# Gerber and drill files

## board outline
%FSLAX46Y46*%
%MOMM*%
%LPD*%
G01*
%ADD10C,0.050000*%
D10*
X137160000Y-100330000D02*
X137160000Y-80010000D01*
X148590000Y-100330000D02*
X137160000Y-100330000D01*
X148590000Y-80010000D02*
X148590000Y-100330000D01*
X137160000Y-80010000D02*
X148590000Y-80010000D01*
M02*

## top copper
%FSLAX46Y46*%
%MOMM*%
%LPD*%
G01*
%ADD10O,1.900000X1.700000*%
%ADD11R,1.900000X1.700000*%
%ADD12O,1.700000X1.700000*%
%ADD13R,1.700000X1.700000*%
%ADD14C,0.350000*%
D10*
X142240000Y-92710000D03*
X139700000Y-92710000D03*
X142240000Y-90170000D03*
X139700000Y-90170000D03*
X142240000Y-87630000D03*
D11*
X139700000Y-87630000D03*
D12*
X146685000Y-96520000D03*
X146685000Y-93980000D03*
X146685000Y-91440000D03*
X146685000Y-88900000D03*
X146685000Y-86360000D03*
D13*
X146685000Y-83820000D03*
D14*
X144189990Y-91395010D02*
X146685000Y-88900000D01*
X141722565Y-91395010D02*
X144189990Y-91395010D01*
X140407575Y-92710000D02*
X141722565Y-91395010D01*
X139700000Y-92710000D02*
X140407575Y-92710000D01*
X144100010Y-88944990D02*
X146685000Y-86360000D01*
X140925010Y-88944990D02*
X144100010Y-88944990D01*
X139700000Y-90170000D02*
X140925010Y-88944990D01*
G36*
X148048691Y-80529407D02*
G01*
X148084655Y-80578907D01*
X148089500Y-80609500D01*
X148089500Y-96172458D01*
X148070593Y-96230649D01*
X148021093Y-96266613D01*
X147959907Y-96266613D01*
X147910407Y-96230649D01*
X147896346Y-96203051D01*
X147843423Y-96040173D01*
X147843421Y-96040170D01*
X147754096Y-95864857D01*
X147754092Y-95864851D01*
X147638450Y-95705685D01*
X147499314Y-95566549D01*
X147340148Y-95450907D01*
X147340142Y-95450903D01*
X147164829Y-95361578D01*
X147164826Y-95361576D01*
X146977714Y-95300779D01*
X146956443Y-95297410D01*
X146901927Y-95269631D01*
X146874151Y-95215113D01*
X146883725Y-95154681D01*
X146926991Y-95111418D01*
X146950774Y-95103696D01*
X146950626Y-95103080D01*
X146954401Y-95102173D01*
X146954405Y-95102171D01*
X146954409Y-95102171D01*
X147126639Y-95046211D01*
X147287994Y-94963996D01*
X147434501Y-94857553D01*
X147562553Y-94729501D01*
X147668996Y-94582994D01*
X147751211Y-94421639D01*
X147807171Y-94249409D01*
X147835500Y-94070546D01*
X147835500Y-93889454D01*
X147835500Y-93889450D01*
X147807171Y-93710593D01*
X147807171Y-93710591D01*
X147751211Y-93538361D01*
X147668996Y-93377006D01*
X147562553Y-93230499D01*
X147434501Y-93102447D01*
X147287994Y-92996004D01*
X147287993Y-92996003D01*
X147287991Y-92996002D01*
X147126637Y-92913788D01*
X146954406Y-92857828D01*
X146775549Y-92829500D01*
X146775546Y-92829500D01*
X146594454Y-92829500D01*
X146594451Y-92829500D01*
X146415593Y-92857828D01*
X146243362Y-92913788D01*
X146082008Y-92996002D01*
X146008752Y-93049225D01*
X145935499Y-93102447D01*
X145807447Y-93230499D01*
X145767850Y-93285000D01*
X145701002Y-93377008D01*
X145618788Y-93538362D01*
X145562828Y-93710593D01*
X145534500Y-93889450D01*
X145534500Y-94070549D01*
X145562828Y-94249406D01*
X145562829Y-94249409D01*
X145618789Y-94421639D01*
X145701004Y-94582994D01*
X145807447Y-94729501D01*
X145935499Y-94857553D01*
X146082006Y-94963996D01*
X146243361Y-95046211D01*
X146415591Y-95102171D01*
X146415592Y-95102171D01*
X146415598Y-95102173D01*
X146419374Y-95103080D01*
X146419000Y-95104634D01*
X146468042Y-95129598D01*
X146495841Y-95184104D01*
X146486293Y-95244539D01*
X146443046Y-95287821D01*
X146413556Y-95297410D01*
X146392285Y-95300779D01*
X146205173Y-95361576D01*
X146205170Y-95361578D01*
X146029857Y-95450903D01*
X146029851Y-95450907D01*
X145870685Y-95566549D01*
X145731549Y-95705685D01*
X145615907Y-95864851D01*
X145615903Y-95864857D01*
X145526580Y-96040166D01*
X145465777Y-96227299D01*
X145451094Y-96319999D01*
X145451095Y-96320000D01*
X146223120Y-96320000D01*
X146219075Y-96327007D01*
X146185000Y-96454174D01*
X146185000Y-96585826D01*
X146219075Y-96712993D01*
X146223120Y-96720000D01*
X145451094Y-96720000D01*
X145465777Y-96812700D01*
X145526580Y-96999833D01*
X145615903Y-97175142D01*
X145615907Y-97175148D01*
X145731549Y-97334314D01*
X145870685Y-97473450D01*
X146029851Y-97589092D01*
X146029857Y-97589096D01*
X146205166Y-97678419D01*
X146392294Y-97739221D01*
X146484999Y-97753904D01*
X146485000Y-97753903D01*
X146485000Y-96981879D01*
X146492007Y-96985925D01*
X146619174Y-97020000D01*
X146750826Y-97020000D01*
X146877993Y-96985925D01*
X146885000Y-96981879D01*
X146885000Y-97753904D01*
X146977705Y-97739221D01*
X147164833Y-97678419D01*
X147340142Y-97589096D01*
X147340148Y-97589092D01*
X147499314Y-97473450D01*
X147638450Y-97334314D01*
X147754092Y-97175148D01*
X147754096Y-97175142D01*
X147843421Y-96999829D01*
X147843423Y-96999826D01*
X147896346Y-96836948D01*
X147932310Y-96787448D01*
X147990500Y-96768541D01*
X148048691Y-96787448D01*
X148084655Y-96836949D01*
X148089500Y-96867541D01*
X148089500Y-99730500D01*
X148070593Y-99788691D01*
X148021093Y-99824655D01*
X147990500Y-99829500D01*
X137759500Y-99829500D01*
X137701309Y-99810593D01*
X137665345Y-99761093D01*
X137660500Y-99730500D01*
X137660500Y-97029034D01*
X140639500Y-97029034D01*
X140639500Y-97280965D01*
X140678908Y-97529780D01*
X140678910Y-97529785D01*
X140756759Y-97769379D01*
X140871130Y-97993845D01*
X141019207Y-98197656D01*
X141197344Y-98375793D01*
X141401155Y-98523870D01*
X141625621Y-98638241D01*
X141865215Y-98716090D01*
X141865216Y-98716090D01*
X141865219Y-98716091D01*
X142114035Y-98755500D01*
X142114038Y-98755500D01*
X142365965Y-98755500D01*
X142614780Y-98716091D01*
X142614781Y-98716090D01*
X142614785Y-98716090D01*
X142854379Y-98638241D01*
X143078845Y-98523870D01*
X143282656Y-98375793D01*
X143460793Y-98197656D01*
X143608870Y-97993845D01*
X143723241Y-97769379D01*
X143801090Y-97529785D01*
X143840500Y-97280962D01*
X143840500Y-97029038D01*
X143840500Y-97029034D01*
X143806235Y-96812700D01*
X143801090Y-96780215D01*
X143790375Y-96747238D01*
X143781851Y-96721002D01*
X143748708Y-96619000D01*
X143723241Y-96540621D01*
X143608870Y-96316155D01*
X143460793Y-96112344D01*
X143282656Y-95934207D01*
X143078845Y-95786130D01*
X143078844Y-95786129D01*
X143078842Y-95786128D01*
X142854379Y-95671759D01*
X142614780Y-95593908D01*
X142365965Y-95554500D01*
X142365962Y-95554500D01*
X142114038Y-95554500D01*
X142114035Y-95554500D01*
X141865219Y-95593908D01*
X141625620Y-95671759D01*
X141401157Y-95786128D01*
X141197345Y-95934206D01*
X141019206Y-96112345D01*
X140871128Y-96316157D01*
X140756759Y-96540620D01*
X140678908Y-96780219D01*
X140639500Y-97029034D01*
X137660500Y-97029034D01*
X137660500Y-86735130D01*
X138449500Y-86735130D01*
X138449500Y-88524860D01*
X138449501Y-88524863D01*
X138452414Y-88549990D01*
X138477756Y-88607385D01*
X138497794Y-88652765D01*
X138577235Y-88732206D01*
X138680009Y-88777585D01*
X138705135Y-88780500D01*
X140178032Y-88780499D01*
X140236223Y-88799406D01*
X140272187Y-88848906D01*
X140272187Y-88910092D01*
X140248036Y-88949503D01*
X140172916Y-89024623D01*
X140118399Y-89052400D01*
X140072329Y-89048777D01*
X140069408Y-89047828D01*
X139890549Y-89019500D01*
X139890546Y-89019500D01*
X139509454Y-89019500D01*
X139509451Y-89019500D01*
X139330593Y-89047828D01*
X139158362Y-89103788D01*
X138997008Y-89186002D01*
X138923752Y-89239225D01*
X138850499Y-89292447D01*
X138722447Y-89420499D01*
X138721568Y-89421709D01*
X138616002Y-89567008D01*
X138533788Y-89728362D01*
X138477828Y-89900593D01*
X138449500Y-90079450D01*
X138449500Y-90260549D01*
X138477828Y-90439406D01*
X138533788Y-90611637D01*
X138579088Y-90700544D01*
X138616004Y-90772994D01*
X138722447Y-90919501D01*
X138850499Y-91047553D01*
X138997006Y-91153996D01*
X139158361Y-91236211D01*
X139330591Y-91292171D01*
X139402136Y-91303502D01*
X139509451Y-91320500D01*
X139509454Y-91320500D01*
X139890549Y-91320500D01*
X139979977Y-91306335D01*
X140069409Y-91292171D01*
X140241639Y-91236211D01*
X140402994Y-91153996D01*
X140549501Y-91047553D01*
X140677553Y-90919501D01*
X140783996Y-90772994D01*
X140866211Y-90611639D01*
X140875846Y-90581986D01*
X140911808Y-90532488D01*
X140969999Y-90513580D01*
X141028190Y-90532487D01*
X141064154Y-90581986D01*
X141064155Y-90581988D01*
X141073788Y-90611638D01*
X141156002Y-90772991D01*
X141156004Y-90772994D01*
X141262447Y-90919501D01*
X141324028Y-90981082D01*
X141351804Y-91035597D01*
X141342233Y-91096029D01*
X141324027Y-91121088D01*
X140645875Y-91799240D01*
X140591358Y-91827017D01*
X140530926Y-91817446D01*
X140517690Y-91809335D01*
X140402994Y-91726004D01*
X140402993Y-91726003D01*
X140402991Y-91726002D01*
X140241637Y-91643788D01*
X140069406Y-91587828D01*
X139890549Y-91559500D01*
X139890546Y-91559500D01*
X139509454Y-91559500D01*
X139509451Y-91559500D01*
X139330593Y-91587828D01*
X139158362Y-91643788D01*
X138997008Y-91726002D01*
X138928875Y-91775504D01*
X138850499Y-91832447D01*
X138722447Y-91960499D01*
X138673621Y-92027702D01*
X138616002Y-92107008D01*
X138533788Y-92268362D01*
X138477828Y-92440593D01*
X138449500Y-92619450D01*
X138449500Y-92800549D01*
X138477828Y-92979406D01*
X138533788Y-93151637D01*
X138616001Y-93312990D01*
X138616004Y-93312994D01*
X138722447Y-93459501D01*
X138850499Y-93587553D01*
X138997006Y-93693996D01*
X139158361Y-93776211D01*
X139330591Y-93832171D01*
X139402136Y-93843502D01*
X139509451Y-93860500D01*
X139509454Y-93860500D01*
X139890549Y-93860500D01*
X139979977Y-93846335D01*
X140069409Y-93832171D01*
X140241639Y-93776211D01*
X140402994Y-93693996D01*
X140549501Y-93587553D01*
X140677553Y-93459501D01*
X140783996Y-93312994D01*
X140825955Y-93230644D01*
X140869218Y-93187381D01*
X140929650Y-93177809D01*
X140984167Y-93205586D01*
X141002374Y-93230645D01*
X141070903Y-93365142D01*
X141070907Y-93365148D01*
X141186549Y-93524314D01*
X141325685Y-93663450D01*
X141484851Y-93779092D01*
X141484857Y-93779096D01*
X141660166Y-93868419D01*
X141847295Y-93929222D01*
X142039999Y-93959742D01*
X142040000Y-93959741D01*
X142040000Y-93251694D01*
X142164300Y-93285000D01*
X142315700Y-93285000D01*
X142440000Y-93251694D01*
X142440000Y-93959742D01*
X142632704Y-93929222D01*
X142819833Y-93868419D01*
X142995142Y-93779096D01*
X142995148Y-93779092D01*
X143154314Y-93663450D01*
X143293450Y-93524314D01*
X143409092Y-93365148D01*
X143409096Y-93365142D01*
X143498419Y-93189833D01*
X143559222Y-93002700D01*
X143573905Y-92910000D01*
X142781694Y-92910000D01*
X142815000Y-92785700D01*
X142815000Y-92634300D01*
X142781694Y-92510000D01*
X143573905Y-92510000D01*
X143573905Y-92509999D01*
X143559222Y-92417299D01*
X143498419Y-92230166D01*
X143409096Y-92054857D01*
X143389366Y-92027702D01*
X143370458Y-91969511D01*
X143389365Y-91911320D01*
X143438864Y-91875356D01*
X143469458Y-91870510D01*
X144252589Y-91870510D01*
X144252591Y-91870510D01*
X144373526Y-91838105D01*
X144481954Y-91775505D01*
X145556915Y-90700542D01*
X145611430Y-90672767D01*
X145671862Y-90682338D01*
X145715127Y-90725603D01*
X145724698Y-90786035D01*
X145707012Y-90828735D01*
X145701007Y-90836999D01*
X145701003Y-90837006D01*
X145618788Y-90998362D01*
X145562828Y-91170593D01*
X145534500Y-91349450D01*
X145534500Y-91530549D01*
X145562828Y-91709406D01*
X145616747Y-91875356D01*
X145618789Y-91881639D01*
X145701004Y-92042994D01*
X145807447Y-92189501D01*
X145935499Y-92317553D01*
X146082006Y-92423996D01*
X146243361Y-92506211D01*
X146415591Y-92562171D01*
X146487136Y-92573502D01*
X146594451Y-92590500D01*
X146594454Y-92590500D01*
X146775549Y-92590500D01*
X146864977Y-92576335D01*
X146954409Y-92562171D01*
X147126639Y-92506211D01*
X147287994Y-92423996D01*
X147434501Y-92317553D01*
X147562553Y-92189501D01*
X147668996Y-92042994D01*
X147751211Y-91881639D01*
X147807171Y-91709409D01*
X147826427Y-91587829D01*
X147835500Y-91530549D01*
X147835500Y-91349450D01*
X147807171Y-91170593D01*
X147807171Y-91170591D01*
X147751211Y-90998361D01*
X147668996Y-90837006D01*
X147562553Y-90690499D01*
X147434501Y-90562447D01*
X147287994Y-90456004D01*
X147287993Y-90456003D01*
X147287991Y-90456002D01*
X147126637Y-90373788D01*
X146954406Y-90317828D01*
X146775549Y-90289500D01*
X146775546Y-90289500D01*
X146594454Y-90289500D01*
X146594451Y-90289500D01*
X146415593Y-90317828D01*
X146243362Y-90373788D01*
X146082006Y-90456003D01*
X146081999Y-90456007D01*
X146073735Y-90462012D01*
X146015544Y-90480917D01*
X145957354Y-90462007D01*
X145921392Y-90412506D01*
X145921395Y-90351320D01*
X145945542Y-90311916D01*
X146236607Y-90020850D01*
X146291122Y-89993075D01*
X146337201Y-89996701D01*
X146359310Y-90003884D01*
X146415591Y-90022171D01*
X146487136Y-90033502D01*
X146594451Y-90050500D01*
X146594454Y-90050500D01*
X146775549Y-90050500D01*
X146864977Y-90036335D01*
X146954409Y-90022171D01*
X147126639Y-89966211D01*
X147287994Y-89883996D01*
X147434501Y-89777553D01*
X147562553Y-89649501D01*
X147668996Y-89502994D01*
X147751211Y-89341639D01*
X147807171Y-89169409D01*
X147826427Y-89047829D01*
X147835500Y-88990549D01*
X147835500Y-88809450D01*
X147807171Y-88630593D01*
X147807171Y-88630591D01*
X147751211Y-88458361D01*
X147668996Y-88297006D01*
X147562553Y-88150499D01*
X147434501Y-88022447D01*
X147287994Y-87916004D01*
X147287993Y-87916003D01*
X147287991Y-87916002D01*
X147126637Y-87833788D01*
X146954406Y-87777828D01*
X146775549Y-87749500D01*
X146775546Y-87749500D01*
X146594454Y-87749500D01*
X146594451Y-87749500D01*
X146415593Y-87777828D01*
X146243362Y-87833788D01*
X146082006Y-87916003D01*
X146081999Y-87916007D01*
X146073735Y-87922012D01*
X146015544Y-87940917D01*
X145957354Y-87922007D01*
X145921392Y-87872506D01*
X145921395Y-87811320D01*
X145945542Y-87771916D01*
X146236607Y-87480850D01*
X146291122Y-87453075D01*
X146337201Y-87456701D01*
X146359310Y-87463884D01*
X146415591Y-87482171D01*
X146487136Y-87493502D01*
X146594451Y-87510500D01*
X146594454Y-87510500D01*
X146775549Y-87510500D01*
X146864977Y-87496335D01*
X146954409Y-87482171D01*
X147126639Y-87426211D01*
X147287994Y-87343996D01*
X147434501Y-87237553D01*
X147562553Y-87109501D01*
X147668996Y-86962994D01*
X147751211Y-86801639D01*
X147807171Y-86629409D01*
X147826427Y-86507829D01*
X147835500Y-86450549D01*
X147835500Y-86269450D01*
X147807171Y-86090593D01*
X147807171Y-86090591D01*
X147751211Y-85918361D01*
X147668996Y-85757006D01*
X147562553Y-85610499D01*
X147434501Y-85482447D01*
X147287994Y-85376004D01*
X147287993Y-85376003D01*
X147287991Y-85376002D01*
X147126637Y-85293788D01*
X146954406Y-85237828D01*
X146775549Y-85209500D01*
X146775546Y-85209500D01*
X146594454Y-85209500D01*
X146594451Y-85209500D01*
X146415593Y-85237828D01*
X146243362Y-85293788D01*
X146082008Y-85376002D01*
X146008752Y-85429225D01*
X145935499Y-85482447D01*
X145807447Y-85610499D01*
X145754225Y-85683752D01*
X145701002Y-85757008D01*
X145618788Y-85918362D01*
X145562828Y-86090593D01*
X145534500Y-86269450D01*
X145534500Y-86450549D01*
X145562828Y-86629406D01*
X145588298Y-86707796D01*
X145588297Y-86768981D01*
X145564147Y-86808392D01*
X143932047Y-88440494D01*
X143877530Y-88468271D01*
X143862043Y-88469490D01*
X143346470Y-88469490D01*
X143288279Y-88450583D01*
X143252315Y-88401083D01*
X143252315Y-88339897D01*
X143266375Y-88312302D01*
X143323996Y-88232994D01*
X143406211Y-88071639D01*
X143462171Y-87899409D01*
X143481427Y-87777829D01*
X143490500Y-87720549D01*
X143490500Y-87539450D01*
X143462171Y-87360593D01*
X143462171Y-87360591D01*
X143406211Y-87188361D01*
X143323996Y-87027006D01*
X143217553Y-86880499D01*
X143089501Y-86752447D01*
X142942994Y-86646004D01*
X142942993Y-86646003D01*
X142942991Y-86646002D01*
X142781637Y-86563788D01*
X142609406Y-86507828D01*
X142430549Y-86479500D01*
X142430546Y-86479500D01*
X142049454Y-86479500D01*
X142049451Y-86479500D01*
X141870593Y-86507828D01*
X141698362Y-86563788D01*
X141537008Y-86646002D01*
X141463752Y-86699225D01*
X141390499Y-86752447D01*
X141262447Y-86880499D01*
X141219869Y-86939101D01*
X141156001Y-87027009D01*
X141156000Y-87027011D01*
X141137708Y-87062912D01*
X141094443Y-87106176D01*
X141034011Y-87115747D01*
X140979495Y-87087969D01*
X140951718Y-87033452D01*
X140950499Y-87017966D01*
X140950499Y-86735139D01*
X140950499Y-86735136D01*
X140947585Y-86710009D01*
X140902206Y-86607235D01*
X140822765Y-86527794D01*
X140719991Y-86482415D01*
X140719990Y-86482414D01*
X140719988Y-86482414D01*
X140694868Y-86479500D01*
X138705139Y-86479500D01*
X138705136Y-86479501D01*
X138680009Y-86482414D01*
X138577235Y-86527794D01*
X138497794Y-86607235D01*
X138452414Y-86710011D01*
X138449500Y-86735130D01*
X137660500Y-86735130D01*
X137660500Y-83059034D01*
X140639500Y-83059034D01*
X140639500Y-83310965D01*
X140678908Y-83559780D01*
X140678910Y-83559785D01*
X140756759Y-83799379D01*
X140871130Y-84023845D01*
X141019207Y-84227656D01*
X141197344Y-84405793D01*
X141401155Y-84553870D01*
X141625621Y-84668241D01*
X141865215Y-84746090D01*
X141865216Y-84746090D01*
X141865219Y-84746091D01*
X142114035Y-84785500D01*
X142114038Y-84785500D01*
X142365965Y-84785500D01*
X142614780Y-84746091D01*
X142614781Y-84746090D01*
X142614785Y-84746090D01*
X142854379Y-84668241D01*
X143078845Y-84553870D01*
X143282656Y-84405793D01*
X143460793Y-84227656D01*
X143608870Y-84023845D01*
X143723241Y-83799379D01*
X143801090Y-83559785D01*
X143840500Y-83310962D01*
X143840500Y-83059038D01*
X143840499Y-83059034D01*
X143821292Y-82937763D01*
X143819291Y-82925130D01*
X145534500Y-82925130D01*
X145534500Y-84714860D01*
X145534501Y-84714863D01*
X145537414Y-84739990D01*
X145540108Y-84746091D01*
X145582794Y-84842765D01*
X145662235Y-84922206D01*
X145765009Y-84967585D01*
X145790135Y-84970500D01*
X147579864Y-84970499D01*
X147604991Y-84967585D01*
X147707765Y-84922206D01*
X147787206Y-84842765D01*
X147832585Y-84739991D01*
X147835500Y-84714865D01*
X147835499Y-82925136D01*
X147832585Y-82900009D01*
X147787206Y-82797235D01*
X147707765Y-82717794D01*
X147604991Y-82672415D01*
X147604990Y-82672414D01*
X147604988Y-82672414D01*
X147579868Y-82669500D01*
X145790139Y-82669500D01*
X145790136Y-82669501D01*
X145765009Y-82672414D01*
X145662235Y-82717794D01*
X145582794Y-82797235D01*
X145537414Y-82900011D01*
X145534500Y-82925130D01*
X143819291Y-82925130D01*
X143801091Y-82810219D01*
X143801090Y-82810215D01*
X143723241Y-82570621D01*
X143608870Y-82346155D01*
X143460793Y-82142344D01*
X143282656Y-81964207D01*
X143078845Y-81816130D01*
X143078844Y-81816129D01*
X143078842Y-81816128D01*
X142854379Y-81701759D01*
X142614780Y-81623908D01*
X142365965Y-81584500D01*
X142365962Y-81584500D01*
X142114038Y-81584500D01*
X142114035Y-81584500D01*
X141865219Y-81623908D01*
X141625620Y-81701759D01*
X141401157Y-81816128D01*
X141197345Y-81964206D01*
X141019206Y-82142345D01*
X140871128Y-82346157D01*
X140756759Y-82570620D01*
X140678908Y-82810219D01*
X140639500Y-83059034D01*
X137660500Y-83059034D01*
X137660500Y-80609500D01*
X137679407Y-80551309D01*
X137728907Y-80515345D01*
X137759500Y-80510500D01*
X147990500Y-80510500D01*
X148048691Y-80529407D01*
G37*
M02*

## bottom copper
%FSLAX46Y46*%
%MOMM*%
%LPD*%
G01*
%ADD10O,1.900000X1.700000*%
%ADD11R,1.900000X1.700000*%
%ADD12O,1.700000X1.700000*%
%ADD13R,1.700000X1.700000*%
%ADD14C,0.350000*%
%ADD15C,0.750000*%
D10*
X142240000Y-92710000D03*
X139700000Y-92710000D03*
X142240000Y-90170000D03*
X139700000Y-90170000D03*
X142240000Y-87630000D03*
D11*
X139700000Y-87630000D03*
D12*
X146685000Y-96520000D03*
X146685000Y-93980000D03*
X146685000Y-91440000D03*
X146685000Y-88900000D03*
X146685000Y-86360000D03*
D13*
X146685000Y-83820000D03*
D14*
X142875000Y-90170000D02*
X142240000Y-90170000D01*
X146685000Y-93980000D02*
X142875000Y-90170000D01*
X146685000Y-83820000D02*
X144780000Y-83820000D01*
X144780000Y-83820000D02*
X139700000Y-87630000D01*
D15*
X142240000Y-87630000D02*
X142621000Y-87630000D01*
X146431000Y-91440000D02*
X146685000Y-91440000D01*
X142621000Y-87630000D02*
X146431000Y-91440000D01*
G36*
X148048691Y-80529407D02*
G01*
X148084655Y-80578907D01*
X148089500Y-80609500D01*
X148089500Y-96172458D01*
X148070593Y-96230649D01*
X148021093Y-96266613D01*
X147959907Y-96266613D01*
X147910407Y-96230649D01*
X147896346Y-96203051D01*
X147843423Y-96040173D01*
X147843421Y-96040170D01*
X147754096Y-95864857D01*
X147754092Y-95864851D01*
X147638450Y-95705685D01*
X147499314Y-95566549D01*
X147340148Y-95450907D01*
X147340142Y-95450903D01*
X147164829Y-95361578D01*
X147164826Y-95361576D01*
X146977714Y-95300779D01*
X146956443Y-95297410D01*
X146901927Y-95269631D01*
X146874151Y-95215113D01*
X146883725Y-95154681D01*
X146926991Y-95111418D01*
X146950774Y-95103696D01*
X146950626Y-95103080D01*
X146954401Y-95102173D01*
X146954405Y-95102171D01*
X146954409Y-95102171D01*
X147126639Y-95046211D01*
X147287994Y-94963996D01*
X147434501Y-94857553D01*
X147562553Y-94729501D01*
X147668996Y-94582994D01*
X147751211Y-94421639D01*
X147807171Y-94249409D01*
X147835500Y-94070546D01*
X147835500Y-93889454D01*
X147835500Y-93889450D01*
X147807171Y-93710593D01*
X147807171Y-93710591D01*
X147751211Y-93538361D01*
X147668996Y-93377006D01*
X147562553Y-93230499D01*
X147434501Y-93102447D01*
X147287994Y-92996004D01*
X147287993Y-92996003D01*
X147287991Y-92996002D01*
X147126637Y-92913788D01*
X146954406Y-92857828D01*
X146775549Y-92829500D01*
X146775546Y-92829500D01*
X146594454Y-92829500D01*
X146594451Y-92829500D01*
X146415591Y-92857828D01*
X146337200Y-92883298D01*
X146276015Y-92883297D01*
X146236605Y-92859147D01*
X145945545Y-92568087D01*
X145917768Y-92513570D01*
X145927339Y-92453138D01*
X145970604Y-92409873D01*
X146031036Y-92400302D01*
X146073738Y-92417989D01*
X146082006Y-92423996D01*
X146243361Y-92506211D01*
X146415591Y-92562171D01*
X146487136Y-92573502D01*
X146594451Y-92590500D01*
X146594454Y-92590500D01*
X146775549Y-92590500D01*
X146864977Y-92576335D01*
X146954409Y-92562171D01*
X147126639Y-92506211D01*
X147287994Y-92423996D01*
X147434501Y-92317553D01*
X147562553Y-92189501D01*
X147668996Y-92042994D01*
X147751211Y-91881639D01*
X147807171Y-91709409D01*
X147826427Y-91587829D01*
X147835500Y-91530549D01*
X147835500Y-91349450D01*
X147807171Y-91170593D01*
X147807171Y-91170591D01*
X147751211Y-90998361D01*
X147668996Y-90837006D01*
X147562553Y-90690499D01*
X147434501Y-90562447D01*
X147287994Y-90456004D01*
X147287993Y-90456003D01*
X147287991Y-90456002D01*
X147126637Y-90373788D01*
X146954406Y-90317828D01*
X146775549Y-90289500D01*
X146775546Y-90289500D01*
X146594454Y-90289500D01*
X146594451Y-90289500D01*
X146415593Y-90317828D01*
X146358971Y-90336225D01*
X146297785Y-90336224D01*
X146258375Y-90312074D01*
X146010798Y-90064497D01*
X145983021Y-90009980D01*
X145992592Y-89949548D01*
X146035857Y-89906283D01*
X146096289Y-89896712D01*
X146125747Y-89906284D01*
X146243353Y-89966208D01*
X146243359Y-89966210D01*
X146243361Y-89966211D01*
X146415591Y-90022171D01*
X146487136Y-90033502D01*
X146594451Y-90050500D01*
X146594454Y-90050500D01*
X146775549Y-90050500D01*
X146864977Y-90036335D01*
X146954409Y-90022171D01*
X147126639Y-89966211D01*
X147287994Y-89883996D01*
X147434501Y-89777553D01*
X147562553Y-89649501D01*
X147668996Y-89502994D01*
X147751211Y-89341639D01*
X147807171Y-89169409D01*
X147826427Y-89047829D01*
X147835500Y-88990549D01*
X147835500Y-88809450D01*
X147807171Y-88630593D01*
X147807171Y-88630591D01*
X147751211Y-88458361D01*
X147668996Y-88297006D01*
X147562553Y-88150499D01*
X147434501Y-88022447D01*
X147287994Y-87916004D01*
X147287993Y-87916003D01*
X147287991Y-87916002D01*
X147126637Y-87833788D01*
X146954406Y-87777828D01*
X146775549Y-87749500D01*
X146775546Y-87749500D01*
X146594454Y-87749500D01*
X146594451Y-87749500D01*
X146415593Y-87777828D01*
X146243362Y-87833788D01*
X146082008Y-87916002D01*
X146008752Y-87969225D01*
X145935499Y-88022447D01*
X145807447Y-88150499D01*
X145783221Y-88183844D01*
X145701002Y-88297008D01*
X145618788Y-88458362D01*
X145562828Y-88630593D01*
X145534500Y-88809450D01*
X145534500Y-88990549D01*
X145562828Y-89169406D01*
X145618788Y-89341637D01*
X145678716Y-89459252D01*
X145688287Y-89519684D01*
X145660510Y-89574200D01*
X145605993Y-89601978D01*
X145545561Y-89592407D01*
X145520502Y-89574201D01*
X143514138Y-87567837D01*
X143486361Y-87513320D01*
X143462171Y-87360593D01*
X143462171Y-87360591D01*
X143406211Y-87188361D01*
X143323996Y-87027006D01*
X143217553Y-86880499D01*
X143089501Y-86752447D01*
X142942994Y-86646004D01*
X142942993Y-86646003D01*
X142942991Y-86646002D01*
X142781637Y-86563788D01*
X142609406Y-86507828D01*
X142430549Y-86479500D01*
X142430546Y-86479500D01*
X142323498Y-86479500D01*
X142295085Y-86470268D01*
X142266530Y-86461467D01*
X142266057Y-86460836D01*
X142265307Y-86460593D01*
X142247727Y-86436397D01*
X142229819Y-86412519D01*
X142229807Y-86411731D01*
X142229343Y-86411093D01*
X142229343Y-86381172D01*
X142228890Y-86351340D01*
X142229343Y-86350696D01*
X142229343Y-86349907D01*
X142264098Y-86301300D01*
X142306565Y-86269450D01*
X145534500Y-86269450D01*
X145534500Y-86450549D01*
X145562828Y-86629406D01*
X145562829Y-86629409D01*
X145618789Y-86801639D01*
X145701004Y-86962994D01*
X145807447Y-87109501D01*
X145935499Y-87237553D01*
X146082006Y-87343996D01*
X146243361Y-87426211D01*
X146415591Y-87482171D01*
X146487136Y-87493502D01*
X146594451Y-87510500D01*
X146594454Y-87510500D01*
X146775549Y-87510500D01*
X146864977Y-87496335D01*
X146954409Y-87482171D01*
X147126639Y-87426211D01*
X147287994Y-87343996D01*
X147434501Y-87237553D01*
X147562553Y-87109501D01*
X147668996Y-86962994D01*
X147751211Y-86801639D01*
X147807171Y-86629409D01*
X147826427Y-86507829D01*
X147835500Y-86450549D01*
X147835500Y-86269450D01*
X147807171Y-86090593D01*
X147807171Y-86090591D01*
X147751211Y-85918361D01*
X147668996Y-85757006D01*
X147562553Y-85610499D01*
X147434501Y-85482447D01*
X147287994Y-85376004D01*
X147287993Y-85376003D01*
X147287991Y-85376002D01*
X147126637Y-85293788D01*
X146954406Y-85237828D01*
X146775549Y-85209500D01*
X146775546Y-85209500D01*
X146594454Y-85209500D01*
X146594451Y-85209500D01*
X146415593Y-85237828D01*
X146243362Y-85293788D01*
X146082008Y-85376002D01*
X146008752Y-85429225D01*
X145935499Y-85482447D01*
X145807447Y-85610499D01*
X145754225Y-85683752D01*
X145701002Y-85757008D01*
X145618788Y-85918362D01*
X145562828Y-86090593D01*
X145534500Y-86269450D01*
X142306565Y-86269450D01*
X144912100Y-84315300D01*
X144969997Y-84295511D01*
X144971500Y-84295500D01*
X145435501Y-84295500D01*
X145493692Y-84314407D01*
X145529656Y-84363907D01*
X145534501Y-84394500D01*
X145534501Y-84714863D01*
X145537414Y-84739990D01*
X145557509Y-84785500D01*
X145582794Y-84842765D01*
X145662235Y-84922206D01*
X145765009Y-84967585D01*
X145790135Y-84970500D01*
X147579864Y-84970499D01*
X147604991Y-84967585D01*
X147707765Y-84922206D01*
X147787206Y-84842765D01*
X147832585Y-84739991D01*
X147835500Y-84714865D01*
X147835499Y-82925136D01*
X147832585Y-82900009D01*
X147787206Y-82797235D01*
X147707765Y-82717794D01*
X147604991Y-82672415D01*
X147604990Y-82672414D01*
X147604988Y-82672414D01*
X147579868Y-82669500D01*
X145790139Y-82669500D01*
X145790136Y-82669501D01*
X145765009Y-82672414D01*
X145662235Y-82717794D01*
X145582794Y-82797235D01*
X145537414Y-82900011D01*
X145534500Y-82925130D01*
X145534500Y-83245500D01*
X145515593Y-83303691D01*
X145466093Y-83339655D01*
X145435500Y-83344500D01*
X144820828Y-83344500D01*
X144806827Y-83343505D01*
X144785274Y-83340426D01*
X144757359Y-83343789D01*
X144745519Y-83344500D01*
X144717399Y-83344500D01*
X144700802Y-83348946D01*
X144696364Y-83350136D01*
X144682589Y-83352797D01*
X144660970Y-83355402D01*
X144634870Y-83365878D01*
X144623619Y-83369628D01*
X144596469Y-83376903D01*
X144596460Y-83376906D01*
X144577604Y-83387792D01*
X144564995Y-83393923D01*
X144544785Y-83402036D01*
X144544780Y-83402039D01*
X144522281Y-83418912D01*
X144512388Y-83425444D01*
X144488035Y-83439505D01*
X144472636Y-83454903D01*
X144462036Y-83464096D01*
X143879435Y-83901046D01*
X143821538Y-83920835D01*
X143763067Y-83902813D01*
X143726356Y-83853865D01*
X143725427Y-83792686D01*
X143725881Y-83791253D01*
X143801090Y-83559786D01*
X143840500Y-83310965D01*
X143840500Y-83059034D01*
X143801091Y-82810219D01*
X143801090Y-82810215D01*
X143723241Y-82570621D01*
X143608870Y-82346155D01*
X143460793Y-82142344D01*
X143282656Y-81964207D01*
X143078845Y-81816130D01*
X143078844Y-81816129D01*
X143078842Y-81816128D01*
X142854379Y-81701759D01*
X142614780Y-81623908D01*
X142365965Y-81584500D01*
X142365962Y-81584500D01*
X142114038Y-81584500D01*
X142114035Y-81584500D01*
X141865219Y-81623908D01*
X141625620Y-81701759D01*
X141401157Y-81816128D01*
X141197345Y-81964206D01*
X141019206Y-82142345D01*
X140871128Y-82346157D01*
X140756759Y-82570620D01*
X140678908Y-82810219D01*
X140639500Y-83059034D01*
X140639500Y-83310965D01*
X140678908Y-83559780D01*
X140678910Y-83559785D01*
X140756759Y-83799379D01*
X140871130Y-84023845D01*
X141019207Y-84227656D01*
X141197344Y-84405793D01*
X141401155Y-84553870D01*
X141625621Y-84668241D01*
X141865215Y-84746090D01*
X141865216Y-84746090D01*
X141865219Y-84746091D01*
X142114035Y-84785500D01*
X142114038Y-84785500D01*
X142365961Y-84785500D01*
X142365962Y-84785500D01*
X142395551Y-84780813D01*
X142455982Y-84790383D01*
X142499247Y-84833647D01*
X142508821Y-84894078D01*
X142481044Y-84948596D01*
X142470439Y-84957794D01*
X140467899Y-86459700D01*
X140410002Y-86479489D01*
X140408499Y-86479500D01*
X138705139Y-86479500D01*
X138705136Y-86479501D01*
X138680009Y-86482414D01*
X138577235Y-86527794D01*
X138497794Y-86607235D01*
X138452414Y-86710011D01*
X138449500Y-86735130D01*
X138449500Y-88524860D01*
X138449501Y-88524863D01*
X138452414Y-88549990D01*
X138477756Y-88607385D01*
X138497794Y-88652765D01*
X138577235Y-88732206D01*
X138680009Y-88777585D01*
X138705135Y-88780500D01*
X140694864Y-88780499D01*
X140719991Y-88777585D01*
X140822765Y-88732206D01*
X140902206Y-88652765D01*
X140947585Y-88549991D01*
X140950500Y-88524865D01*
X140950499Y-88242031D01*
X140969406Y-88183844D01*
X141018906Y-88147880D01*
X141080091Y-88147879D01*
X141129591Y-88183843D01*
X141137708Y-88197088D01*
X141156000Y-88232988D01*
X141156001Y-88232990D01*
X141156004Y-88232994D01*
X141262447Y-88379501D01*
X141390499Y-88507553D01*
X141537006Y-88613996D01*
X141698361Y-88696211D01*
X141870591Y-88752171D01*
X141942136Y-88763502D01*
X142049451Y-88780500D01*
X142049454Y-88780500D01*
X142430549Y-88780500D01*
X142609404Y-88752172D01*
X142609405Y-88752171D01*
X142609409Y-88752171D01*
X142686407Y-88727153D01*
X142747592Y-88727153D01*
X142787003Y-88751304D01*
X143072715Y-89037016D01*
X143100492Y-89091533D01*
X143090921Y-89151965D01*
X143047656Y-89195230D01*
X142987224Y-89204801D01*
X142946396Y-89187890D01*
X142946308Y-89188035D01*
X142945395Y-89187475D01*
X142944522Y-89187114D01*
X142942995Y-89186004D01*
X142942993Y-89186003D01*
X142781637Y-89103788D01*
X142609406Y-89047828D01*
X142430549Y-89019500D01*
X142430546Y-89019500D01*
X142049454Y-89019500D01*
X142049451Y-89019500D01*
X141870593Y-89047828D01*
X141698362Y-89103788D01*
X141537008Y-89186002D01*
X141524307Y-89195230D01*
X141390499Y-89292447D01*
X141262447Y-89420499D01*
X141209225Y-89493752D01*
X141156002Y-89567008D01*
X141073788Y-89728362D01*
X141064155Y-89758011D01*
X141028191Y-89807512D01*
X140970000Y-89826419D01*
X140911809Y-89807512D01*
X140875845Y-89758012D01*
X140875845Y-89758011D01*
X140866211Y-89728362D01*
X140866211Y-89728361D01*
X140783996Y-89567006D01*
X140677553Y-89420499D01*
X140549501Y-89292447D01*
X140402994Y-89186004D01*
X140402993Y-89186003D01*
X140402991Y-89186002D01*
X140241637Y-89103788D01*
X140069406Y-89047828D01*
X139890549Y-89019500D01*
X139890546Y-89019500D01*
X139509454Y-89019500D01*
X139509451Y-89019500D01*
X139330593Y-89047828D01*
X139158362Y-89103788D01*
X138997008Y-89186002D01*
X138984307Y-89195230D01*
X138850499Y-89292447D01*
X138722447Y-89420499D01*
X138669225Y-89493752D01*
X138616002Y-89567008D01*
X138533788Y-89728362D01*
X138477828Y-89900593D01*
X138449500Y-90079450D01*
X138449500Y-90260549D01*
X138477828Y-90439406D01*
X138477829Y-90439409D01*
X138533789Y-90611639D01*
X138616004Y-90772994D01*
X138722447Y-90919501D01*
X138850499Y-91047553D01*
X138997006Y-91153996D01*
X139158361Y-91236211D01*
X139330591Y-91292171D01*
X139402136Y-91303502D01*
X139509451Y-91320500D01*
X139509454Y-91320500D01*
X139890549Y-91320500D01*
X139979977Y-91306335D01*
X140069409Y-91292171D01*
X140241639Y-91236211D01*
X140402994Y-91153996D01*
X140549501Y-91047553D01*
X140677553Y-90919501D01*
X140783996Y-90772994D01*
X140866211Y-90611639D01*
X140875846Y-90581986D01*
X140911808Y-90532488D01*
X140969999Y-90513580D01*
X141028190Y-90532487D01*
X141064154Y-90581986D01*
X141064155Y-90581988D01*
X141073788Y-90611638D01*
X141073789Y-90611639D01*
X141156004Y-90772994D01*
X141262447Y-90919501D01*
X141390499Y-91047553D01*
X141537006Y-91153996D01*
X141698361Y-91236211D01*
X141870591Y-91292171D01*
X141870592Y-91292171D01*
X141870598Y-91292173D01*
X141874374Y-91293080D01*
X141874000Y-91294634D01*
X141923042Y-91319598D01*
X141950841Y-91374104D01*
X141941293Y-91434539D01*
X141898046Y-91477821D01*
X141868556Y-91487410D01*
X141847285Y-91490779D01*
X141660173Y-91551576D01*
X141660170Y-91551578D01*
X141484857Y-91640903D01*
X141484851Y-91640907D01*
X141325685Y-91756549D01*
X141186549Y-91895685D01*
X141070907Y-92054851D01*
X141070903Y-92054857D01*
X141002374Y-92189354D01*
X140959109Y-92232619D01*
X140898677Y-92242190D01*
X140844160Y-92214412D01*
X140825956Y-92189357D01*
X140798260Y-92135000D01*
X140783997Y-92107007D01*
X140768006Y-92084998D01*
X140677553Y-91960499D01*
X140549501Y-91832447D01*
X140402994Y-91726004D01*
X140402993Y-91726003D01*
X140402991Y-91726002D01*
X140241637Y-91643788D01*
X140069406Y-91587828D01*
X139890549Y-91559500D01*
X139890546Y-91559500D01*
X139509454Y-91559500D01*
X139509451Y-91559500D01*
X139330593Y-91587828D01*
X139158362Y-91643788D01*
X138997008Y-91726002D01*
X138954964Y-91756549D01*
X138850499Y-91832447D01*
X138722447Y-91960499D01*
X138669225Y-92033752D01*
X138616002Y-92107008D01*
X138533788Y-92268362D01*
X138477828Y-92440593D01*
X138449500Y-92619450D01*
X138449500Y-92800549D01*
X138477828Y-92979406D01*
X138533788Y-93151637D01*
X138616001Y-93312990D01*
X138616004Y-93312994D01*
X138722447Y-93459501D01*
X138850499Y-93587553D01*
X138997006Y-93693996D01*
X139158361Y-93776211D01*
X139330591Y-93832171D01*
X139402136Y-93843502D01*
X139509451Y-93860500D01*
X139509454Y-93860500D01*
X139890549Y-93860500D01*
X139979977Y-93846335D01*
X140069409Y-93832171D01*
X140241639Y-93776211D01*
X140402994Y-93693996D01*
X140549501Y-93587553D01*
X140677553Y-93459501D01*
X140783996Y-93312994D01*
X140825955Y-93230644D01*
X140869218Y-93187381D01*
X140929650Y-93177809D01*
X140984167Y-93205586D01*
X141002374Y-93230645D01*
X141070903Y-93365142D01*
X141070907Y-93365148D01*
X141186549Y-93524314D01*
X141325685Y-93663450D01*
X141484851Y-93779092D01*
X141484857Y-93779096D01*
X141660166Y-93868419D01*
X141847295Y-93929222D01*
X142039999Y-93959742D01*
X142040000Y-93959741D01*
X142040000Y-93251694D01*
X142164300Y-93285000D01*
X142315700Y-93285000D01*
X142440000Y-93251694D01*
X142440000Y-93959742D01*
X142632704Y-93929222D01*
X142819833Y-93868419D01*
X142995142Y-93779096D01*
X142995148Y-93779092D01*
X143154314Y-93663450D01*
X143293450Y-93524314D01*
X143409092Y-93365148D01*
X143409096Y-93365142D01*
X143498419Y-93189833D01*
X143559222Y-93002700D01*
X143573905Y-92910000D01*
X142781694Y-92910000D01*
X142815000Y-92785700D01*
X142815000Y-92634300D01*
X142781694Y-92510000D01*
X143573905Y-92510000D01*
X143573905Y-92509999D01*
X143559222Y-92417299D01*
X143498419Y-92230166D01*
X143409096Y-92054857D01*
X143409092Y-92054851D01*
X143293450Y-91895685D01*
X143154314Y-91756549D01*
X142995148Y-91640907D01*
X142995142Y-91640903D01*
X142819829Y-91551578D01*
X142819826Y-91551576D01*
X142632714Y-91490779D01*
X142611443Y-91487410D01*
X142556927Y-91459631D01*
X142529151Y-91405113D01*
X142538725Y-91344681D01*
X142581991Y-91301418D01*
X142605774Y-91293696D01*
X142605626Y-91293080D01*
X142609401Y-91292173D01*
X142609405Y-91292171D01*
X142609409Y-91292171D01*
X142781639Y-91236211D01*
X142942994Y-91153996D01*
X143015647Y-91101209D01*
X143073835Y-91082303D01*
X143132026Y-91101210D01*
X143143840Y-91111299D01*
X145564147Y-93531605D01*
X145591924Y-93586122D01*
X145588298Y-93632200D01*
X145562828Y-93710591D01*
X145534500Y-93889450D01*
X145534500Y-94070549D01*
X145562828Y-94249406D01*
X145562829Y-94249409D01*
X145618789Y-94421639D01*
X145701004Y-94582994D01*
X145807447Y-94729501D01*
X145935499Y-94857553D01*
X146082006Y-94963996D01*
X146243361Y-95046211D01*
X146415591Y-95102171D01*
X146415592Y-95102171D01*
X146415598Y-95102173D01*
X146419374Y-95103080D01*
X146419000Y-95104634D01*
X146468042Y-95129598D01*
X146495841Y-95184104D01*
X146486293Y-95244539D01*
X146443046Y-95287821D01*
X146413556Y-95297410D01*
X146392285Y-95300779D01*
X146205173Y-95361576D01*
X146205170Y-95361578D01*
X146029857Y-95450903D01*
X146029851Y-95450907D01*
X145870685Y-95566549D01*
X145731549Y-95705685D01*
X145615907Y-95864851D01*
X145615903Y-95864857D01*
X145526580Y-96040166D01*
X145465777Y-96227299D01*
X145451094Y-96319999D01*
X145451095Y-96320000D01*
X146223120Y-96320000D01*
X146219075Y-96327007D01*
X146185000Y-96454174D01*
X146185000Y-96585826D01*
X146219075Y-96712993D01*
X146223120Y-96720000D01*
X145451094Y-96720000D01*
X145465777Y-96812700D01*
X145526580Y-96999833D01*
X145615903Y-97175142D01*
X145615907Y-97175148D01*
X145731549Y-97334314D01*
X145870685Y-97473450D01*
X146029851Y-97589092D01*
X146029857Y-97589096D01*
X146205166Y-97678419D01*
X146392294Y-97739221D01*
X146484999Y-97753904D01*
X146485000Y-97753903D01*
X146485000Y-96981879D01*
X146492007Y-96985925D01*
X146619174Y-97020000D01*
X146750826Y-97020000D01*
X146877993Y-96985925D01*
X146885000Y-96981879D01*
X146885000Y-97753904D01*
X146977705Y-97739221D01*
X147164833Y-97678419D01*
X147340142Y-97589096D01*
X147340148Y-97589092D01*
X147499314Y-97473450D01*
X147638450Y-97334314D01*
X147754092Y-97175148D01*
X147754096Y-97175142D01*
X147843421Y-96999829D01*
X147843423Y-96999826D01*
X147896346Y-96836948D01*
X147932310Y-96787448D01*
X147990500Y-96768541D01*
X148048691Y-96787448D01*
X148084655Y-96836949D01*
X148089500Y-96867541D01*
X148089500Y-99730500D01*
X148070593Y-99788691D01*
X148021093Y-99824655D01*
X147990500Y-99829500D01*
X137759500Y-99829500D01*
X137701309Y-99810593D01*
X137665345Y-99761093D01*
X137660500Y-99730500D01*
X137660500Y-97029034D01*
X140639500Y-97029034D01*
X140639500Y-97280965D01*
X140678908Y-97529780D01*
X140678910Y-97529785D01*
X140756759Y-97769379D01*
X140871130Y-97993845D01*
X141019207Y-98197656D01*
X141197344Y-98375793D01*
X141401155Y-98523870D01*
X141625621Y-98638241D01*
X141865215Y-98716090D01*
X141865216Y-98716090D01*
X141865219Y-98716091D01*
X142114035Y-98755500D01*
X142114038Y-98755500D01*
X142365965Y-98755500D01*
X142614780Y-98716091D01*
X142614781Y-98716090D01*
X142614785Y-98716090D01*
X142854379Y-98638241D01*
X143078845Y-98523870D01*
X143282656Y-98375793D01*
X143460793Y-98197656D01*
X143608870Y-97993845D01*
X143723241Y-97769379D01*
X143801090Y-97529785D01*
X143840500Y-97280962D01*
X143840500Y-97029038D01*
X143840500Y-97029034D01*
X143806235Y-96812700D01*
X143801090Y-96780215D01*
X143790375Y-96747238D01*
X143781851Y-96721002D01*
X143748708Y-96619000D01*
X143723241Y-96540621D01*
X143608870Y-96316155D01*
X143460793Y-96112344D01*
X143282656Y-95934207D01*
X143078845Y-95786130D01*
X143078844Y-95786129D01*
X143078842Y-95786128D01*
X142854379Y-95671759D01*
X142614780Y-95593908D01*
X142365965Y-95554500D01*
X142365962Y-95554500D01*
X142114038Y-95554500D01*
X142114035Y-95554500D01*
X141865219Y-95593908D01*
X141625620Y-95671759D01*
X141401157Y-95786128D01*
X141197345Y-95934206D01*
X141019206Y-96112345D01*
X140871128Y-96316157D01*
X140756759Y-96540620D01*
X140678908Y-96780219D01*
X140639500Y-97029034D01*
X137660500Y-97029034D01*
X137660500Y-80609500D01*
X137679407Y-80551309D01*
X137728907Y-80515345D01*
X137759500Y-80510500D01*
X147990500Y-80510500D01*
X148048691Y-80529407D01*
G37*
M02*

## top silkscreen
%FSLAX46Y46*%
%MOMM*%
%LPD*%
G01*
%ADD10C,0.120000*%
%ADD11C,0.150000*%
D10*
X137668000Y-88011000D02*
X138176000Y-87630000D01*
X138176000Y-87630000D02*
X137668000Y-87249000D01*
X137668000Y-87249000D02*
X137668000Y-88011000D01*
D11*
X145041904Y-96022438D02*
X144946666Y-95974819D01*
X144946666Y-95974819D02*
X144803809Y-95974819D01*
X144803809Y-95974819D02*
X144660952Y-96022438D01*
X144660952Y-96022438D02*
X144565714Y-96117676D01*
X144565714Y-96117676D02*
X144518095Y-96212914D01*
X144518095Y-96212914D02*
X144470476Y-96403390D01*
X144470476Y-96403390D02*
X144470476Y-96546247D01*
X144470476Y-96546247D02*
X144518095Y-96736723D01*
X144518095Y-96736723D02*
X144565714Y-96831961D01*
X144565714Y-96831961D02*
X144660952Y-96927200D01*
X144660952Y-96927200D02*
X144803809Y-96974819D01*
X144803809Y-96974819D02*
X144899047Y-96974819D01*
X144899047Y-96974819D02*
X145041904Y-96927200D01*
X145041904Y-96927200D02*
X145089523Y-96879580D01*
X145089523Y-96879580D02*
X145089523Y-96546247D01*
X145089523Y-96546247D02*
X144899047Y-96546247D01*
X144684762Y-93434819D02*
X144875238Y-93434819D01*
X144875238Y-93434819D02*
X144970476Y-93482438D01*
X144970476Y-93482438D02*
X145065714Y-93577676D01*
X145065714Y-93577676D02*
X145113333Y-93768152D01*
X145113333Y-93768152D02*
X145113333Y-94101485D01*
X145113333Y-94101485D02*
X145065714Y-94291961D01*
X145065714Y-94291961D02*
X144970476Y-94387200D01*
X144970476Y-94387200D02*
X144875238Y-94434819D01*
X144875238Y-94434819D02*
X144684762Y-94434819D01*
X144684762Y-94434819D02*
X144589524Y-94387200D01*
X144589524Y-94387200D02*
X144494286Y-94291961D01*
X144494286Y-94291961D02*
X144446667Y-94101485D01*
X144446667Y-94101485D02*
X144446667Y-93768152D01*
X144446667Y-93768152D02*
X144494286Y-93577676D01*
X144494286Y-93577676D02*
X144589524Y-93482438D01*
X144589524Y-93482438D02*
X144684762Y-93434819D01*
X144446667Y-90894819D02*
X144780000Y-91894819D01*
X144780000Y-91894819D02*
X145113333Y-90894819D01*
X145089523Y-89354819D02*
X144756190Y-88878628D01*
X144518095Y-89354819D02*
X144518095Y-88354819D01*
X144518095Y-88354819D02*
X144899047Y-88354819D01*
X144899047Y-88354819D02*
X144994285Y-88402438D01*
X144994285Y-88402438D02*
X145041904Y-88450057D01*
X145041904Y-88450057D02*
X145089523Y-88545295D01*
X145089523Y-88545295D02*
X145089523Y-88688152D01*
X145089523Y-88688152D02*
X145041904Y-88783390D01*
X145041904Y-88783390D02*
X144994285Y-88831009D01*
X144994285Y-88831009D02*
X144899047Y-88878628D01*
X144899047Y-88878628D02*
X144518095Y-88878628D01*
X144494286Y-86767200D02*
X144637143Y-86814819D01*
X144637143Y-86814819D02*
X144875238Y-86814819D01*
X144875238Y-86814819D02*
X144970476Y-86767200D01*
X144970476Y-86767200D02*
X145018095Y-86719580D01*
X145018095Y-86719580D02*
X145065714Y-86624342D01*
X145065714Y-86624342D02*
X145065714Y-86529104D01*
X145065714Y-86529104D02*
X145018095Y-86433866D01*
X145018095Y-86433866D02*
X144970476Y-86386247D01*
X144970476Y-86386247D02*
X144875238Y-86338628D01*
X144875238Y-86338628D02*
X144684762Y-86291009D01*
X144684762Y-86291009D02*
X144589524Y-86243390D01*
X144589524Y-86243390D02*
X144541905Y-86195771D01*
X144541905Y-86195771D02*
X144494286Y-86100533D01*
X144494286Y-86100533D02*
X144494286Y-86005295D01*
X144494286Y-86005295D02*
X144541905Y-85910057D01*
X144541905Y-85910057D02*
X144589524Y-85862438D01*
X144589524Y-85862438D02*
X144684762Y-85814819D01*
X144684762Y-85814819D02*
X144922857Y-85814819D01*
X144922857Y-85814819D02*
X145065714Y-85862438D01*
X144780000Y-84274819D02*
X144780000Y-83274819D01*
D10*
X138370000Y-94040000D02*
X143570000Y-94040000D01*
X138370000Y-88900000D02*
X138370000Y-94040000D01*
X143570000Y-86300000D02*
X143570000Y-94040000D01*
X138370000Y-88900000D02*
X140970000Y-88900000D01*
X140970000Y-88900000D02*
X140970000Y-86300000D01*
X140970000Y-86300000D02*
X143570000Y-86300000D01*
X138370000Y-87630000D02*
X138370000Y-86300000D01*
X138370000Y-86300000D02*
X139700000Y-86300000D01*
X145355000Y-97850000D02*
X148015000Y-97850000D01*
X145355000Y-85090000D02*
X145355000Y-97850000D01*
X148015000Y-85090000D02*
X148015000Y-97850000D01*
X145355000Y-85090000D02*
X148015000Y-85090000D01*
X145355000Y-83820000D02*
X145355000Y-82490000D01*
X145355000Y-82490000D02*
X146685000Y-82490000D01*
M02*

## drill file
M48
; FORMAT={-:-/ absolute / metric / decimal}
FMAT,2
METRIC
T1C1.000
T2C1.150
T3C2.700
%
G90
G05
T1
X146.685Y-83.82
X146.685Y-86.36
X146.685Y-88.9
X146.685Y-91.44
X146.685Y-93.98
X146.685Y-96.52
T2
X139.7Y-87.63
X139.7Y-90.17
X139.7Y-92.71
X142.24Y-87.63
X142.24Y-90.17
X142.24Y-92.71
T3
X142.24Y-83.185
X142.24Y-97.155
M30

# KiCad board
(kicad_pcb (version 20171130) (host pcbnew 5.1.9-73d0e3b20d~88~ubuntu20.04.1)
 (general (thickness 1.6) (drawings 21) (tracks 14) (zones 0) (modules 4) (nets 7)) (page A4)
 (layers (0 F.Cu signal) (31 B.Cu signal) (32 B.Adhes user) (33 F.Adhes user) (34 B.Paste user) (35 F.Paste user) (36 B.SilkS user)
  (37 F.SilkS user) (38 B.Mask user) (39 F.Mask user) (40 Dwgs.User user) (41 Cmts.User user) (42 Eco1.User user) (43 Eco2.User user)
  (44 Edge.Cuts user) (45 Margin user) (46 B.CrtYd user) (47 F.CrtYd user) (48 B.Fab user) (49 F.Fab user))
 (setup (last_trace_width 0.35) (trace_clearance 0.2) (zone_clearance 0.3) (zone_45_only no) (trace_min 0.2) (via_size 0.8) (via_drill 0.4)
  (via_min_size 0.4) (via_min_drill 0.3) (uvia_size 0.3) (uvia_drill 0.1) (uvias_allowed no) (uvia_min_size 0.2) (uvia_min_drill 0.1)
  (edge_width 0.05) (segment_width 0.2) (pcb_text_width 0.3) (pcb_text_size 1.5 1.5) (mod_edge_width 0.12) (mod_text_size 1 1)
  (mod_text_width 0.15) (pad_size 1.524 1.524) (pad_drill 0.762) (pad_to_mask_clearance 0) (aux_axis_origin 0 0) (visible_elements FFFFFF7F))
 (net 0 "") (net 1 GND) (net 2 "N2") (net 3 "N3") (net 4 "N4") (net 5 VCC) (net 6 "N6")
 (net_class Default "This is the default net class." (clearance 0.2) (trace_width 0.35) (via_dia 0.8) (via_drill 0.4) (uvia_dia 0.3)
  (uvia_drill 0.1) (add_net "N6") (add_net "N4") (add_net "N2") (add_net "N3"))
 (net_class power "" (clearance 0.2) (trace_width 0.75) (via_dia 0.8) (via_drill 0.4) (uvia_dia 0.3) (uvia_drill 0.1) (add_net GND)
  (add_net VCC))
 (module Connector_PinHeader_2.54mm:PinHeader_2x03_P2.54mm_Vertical (layer F.Cu) (at 139.7 87.63)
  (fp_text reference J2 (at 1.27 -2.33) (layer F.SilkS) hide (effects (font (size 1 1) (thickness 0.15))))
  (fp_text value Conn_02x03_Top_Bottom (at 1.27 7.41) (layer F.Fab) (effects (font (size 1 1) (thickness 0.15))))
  (fp_line (start -1.33 6.41) (end 3.87 6.41) (layer F.SilkS) (width 0.12))
  (fp_line (start -1.33 1.27) (end -1.33 6.41) (layer F.SilkS) (width 0.12))
  (fp_line (start 3.87 -1.33) (end 3.87 6.41) (layer F.SilkS) (width 0.12))
  (fp_line (start -1.33 1.27) (end 1.27 1.27) (layer F.SilkS) (width 0.12))
  (fp_line (start 1.27 1.27) (end 1.27 -1.33) (layer F.SilkS) (width 0.12))
  (fp_line (start 1.27 -1.33) (end 3.87 -1.33) (layer F.SilkS) (width 0.12))
  (fp_line (start -1.33 0) (end -1.33 -1.33) (layer F.SilkS) (width 0.12))
  (fp_line (start -1.33 -1.33) (end 0 -1.33) (layer F.SilkS) (width 0.12))
  (pad 6 thru_hole oval (at 2.54 5.08) (size 1.9 1.7) (drill 1.15) (layers *.Cu *.Mask) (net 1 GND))
  (pad 3 thru_hole oval (at 0 5.08) (size 1.9 1.7) (drill 1.15) (layers *.Cu *.Mask) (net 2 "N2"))
  (pad 5 thru_hole oval (at 2.54 2.54) (size 1.9 1.7) (drill 1.15) (layers *.Cu *.Mask) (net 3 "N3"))
  (pad 2 thru_hole oval (at 0 2.54) (size 1.9 1.7) (drill 1.15) (layers *.Cu *.Mask) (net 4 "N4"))
  (pad 4 thru_hole oval (at 2.54 0) (size 1.9 1.7) (drill 1.15) (layers *.Cu *.Mask) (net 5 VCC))
  (pad 1 thru_hole rect (at 0 0) (size 1.9 1.7) (drill 1.15) (layers *.Cu *.Mask) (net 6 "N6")))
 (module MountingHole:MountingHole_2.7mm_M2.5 (layer F.Cu) (at 142.24 97.155)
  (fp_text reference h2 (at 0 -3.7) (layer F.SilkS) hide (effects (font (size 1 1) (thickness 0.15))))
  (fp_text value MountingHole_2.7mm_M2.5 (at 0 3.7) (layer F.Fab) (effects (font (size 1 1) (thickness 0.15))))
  (pad 1 np_thru_hole circle (at 0 0) (size 2.7 2.7) (drill 2.7) (layers *.Cu *.Mask)))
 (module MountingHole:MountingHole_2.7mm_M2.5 (layer F.Cu) (at 142.24 83.185)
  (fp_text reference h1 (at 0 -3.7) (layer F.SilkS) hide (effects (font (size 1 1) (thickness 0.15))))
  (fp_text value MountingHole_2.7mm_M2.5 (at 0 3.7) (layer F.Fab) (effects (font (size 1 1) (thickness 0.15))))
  (pad 1 np_thru_hole circle (at 0 0) (size 2.7 2.7) (drill 2.7) (layers *.Cu *.Mask)))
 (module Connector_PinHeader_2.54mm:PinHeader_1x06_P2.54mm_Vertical (layer F.Cu) (at 146.685 83.82)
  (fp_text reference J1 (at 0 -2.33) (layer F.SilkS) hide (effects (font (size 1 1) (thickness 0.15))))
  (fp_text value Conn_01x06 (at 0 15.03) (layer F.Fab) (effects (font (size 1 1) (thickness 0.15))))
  (fp_line (start -1.33 14.03) (end 1.33 14.03) (layer F.SilkS) (width 0.12))
  (fp_line (start -1.33 1.27) (end -1.33 14.03) (layer F.SilkS) (width 0.12))
  (fp_line (start 1.33 1.27) (end 1.33 14.03) (layer F.SilkS) (width 0.12))
  (fp_line (start -1.33 1.27) (end 1.33 1.27) (layer F.SilkS) (width 0.12))
  (fp_line (start -1.33 0) (end -1.33 -1.33) (layer F.SilkS) (width 0.12))
  (fp_line (start -1.33 -1.33) (end 0 -1.33) (layer F.SilkS) (width 0.12))
  (pad 6 thru_hole oval (at 0 12.7) (size 1.7 1.7) (drill 1) (layers *.Cu *.Mask) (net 1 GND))
  (pad 5 thru_hole oval (at 0 10.16) (size 1.7 1.7) (drill 1) (layers *.Cu *.Mask) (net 3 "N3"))
  (pad 4 thru_hole oval (at 0 7.62) (size 1.7 1.7) (drill 1) (layers *.Cu *.Mask) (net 5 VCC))
  (pad 3 thru_hole oval (at 0 5.08) (size 1.7 1.7) (drill 1) (layers *.Cu *.Mask) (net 2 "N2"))
  (pad 2 thru_hole oval (at 0 2.54) (size 1.7 1.7) (drill 1) (layers *.Cu *.Mask) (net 4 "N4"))
  (pad 1 thru_hole rect (at 0 0) (size 1.7 1.7) (drill 1) (layers *.Cu *.Mask) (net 6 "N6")))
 (gr_line (start 137.668 88.011) (end 138.176 87.63) (layer F.SilkS) (width 0.12))
 (gr_line (start 138.176 87.63) (end 137.668 87.249) (layer F.SilkS) (width 0.12))
 (gr_line (start 137.668 87.249) (end 137.668 88.011) (layer F.SilkS) (width 0.12))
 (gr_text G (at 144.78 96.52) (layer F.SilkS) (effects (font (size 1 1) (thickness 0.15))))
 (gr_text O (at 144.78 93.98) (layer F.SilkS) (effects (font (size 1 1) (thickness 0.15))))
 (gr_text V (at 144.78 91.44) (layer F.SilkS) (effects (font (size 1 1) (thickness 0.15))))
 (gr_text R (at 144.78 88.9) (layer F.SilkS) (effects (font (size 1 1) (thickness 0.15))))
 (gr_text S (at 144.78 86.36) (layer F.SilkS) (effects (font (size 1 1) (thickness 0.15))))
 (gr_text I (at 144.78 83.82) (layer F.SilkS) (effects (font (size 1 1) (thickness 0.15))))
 (gr_line (start 137.16 100.33) (end 137.16 80.01) (layer Edge.Cuts) (width 0.05))
 (gr_line (start 148.59 100.33) (end 137.16 100.33) (layer Edge.Cuts) (width 0.05))
 (gr_line (start 148.59 80.01) (end 148.59 100.33) (layer Edge.Cuts) (width 0.05))
 (gr_line (start 137.16 80.01) (end 148.59 80.01) (layer Edge.Cuts) (width 0.05))
 (segment (start 142.875 90.17) (end 142.24 90.17) (width 0.35) (layer B.Cu) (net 3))
 (segment (start 146.685 93.98) (end 142.875 90.17) (width 0.35) (layer B.Cu) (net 3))
 (segment (start 144.18999 91.39501) (end 146.685 88.9) (width 0.35) (layer F.Cu) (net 2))
 (segment (start 141.722565 91.39501) (end 144.18999 91.39501) (width 0.35) (layer F.Cu) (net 2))
 (segment (start 140.407575 92.71) (end 141.722565 91.39501) (width 0.35) (layer F.Cu) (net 2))
 (segment (start 139.7 92.71) (end 140.407575 92.71) (width 0.35) (layer F.Cu) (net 2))
 (segment (start 144.10001 88.94499) (end 146.685 86.36) (width 0.35) (layer F.Cu) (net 4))
 (segment (start 140.92501 88.94499) (end 144.10001 88.94499) (width 0.35) (layer F.Cu) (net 4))
 (segment (start 139.7 90.17) (end 140.92501 88.94499) (width 0.35) (layer F.Cu) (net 4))
 (segment (start 146.685 83.82) (end 144.78 83.82) (width 0.35) (layer B.Cu) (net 6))
 (segment (start 144.78 83.82) (end 139.7 87.63) (width 0.35) (layer B.Cu) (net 6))
 (segment (start 142.24 87.63) (end 142.621 87.63) (width 0.75) (layer B.Cu) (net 5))
 (segment (start 146.431 91.44) (end 146.685 91.44) (width 0.75) (layer B.Cu) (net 5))
 (segment (start 142.621 87.63) (end 146.431 91.44) (width 0.75) (layer B.Cu) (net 5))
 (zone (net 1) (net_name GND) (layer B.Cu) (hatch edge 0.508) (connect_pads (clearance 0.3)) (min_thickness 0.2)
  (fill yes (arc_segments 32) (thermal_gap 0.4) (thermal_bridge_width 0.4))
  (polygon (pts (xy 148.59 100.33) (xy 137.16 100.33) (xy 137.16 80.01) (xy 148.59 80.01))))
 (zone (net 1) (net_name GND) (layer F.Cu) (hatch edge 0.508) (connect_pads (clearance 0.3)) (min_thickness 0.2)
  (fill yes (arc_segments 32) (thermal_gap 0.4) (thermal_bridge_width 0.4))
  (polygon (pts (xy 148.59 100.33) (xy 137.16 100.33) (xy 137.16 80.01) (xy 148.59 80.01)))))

